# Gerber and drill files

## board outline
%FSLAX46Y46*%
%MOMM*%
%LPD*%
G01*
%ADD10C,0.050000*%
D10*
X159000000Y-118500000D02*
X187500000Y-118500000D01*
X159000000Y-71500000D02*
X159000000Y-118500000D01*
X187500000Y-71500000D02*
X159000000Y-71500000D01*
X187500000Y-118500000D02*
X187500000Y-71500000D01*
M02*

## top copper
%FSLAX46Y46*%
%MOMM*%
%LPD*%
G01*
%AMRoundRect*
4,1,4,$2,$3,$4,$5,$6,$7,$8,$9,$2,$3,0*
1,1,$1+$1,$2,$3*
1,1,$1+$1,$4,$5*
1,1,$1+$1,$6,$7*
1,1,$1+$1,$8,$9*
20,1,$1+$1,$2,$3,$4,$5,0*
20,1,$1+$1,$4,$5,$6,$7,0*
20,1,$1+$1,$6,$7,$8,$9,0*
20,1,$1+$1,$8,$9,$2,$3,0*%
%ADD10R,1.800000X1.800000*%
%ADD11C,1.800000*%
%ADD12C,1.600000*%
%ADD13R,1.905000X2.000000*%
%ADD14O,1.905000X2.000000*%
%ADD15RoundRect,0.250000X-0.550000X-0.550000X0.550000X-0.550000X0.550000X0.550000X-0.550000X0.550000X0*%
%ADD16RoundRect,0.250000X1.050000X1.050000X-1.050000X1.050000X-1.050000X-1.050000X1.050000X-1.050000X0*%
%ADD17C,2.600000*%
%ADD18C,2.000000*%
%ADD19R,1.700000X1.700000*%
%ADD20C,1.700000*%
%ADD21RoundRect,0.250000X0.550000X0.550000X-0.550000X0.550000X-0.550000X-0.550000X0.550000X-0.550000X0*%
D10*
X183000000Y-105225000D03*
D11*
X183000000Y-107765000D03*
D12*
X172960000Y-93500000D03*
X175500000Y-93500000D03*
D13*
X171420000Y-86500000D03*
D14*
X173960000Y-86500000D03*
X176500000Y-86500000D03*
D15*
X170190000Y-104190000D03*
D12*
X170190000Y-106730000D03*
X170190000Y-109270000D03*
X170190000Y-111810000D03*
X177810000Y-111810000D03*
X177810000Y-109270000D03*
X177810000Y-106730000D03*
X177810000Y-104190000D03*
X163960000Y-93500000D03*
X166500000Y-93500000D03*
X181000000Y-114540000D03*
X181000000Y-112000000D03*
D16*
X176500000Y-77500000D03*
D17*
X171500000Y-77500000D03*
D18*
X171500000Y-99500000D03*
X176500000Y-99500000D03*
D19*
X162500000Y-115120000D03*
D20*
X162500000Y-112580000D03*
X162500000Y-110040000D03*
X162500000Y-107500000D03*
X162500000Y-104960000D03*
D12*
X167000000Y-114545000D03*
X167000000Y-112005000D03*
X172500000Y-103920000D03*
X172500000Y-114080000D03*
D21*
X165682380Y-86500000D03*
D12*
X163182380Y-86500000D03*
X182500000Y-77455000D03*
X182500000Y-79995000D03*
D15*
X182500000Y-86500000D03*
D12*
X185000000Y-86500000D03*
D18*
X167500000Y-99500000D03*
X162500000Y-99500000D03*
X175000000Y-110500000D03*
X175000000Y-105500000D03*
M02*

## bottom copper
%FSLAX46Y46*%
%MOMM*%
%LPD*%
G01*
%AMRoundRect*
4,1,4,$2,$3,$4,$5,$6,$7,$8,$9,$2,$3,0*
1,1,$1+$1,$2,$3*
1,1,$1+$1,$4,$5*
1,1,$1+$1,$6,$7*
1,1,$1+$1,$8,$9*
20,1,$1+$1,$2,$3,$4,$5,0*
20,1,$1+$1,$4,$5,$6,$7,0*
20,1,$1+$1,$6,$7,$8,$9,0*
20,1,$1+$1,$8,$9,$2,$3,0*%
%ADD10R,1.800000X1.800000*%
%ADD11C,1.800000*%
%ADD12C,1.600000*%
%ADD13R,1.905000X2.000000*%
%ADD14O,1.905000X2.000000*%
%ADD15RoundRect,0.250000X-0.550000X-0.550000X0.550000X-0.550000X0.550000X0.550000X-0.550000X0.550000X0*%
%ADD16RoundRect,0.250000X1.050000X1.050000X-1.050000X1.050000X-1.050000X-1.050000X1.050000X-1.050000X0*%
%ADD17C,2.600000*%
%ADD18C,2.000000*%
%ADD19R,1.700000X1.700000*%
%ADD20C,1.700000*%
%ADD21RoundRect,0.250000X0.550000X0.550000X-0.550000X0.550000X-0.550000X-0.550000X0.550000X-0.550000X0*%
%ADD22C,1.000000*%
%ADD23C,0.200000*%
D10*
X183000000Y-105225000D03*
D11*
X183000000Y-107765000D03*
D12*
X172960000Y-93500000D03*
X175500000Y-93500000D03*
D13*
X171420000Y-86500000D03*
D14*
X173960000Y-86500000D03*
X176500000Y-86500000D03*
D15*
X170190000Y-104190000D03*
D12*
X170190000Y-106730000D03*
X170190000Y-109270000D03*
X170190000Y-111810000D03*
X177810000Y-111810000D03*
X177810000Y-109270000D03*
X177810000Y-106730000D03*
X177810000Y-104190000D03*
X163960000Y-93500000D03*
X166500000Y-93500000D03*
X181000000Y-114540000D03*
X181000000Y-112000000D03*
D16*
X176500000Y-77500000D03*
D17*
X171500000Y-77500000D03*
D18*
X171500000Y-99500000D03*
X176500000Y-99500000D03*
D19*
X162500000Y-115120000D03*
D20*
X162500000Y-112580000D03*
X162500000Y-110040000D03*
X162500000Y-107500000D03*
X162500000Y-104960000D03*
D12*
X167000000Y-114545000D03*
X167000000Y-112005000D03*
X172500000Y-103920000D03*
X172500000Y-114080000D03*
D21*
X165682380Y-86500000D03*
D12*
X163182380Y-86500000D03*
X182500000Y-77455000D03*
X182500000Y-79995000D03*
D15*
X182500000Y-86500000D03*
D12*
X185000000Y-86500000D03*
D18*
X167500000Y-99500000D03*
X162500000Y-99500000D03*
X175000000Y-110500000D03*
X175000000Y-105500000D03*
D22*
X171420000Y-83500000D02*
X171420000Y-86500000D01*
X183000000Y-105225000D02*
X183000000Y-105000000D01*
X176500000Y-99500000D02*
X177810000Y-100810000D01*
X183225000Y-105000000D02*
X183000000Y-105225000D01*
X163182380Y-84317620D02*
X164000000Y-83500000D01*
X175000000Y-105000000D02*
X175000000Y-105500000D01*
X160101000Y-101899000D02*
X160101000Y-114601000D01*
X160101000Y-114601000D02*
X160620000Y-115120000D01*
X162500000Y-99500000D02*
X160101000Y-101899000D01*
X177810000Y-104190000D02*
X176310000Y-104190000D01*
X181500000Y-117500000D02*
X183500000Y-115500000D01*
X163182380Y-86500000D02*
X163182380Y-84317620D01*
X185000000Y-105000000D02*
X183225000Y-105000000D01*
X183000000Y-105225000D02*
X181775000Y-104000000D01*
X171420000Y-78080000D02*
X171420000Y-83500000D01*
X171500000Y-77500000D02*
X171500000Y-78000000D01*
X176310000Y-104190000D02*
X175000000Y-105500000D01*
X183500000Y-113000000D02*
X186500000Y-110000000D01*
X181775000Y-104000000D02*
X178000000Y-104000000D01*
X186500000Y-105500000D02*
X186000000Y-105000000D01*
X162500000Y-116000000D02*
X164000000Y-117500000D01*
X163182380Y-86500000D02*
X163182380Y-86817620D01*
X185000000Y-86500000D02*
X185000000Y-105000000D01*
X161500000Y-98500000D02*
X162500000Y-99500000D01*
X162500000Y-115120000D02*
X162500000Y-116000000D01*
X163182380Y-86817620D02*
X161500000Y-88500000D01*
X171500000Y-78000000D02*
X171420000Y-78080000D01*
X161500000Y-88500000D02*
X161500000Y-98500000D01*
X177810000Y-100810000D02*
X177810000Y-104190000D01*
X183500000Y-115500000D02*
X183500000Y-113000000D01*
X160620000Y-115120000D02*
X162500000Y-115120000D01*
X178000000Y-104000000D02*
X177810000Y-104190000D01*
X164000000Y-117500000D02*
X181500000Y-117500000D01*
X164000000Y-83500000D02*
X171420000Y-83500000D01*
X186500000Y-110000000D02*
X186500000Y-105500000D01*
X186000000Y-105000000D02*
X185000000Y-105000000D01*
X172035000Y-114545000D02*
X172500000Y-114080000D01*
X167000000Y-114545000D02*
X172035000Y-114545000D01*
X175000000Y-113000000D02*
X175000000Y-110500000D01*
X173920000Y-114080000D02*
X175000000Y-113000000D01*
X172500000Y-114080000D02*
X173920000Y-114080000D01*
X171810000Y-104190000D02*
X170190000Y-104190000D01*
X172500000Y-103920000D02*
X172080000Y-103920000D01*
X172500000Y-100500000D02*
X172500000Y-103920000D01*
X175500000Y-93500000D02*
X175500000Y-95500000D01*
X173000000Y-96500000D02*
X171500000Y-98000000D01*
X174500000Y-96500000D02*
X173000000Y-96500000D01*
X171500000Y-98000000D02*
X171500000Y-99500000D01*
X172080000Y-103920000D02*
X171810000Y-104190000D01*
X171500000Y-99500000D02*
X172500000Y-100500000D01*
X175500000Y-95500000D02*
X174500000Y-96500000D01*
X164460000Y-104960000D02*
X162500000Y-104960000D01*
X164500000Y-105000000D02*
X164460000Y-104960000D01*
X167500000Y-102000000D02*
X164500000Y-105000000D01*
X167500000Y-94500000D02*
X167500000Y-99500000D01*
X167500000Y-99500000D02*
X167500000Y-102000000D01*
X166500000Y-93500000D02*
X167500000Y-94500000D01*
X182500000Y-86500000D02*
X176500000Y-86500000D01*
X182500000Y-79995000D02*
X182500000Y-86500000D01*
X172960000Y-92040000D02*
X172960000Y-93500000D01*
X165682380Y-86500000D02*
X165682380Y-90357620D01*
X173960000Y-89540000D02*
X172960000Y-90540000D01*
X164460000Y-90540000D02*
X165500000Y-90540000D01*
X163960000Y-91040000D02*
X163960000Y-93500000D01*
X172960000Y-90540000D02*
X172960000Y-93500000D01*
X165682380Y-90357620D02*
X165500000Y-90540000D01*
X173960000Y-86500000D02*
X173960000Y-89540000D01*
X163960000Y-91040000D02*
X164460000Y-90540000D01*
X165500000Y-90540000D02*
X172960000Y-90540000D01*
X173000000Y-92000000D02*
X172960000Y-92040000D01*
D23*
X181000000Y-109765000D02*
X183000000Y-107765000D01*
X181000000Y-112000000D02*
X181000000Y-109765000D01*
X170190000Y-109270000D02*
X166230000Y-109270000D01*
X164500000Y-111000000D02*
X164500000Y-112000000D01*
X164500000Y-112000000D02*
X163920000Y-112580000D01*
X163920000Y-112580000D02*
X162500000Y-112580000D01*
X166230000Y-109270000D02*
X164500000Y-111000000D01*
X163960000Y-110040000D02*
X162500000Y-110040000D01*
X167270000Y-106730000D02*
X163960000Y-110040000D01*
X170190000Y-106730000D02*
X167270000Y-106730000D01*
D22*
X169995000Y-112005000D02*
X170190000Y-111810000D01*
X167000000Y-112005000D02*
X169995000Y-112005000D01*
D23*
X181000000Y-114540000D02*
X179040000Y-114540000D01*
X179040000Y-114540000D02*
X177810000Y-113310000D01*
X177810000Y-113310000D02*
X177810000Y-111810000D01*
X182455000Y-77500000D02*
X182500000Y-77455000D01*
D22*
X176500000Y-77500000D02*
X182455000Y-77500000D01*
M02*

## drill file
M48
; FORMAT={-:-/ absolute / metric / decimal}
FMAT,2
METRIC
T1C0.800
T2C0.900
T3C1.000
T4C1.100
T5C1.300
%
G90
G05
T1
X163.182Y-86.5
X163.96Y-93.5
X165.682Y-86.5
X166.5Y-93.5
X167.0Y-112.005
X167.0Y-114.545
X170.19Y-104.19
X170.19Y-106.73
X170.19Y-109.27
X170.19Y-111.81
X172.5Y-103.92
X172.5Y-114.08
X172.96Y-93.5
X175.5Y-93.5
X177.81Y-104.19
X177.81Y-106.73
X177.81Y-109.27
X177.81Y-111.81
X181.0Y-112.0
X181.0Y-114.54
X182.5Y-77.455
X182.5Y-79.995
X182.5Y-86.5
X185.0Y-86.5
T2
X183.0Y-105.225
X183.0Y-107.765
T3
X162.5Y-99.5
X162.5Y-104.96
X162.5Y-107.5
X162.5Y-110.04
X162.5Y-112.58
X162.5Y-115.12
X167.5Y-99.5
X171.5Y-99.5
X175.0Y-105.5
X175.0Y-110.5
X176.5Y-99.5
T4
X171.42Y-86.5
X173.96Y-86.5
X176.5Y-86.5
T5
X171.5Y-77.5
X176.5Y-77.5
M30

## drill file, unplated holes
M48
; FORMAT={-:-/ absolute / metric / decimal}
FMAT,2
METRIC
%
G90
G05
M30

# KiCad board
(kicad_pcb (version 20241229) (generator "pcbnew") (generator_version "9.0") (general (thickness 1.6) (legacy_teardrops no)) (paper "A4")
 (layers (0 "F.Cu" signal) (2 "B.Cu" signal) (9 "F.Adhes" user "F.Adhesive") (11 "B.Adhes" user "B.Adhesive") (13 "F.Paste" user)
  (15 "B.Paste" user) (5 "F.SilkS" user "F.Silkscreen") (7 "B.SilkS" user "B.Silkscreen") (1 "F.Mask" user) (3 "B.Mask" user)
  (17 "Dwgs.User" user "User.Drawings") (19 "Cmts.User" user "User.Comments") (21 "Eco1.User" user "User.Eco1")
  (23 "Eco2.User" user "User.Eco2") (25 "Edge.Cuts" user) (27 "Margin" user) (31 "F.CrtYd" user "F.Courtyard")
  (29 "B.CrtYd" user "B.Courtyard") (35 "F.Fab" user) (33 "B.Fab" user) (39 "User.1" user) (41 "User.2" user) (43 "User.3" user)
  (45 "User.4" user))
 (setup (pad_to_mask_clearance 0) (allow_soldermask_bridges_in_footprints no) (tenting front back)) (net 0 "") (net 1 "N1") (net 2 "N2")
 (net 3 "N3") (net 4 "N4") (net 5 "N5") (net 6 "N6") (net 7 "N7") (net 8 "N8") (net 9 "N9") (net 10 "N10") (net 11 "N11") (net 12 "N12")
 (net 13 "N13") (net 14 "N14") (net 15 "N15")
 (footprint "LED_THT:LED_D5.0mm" (layer "F.Cu") (at 183 105.225 -90)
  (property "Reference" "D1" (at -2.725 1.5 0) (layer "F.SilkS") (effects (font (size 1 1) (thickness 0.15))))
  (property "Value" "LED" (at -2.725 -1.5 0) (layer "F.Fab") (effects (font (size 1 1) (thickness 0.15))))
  (pad "1" thru_hole rect (at 0 0 270) (size 1.8 1.8) (drill 0.9) (layers "*.Cu" "*.Mask") (remove_unused_layers no) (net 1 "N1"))
  (pad "2" thru_hole circle (at 2.54 0 270) (size 1.8 1.8) (drill 0.9) (layers "*.Cu" "*.Mask") (remove_unused_layers no) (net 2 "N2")))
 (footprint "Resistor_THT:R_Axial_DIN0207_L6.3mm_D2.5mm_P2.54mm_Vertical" (layer "F.Cu") (at 172.96 93.5)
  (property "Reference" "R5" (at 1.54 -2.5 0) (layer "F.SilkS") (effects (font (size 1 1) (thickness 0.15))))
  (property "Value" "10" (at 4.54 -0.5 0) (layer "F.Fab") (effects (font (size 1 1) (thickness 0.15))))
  (pad "1" thru_hole circle (at 0 0) (size 1.6 1.6) (drill 0.8) (layers "*.Cu" "*.Mask") (remove_unused_layers no) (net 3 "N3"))
  (pad "2" thru_hole circle (at 2.54 0) (size 1.6 1.6) (drill 0.8) (layers "*.Cu" "*.Mask") (remove_unused_layers no) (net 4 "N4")))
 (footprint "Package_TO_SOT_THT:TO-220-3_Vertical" (layer "F.Cu") (at 171.42 86.5)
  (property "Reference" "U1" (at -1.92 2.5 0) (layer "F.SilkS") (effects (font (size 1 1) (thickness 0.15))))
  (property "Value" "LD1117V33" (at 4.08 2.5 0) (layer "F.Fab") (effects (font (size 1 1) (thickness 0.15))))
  (pad "1" thru_hole rect (at 0 0) (size 1.905 2) (drill 1.1) (layers "*.Cu" "*.Mask") (remove_unused_layers no) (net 1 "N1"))
  (pad "2" thru_hole oval (at 2.54 0) (size 1.905 2) (drill 1.1) (layers "*.Cu" "*.Mask") (remove_unused_layers no) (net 3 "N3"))
  (pad "3" thru_hole oval (at 5.08 0) (size 1.905 2) (drill 1.1) (layers "*.Cu" "*.Mask") (remove_unused_layers no) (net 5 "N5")))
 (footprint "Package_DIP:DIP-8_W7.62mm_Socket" (layer "F.Cu") (at 170.19 104.19)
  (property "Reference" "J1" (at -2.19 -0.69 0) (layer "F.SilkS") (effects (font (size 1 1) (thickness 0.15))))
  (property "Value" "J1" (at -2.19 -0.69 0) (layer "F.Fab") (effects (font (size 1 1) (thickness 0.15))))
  (pad "1" thru_hole roundrect (at 0 0) (size 1.6 1.6) (drill 0.8) (layers "*.Cu" "*.Mask") (remove_unused_layers no)
   (roundrect_rratio 0.15625) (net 4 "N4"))
  (pad "2" thru_hole circle (at 0 2.54) (size 1.6 1.6) (drill 0.8) (layers "*.Cu" "*.Mask") (remove_unused_layers no) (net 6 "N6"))
  (pad "3" thru_hole circle (at 0 5.08) (size 1.6 1.6) (drill 0.8) (layers "*.Cu" "*.Mask") (remove_unused_layers no) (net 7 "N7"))
  (pad "4" thru_hole circle (at 0 7.62) (size 1.6 1.6) (drill 0.8) (layers "*.Cu" "*.Mask") (remove_unused_layers no) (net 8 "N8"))
  (pad "5" thru_hole circle (at 7.62 7.62) (size 1.6 1.6) (drill 0.8) (layers "*.Cu" "*.Mask") (remove_unused_layers no) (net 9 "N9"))
  (pad "6" thru_hole circle (at 7.62 5.08) (size 1.6 1.6) (drill 0.8) (layers "*.Cu" "*.Mask") (remove_unused_layers no) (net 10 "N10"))
  (pad "7" thru_hole circle (at 7.62 2.54) (size 1.6 1.6) (drill 0.8) (layers "*.Cu" "*.Mask") (remove_unused_layers no) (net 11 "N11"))
  (pad "8" thru_hole circle (at 7.62 0) (size 1.6 1.6) (drill 0.8) (layers "*.Cu" "*.Mask") (remove_unused_layers no) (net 1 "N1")))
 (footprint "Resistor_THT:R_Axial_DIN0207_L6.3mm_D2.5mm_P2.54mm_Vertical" (layer "F.Cu") (at 163.96 93.5)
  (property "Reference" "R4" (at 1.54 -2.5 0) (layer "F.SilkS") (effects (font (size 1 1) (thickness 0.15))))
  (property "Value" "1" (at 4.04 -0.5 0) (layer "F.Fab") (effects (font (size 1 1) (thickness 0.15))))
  (pad "1" thru_hole circle (at 0 0) (size 1.6 1.6) (drill 0.8) (layers "*.Cu" "*.Mask") (remove_unused_layers no) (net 3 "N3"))
  (pad "2" thru_hole circle (at 2.54 0) (size 1.6 1.6) (drill 0.8) (layers "*.Cu" "*.Mask") (remove_unused_layers no) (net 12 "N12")))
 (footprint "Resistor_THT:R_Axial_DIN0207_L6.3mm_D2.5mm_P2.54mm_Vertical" (layer "F.Cu") (at 181 114.54 90)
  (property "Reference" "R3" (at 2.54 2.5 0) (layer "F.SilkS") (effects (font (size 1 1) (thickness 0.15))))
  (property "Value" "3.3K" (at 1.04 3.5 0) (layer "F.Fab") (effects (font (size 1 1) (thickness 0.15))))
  (pad "1" thru_hole circle (at 0 0 90) (size 1.6 1.6) (drill 0.8) (layers "*.Cu" "*.Mask") (remove_unused_layers no) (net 9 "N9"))
  (pad "2" thru_hole circle (at 2.54 0 90) (size 1.6 1.6) (drill 0.8) (layers "*.Cu" "*.Mask") (remove_unused_layers no) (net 2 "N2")))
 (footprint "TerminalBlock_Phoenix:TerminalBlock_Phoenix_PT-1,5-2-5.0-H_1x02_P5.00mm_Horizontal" (layer "F.Cu") (at 176.5 77.5 180)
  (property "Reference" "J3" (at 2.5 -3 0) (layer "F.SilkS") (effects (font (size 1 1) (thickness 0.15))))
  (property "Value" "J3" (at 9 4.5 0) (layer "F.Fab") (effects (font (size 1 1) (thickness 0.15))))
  (pad "1" thru_hole roundrect (at 0 0 180) (size 2.6 2.6) (drill 1.3) (layers "*.Cu" "*.Mask") (remove_unused_layers no)
   (roundrect_rratio 0.096154) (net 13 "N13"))
  (pad "2" thru_hole circle (at 5 0 180) (size 2.6 2.6) (drill 1.3) (layers "*.Cu" "*.Mask") (remove_unused_layers no) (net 1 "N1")))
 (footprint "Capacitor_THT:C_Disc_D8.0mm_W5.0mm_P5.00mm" (layer "F.Cu") (at 171.5 99.5)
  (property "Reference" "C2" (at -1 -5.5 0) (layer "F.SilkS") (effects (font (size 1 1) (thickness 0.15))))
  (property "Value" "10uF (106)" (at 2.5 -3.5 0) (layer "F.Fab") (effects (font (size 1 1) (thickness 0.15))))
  (pad "1" thru_hole circle (at 0 0) (size 2 2) (drill 1) (layers "*.Cu" "*.Mask") (remove_unused_layers no) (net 4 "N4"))
  (pad "2" thru_hole circle (at 5 0) (size 2 2) (drill 1) (layers "*.Cu" "*.Mask") (remove_unused_layers no) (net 1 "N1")))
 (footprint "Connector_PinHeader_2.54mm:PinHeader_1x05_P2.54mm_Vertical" (layer "F.Cu") (at 162.5 115.12 180)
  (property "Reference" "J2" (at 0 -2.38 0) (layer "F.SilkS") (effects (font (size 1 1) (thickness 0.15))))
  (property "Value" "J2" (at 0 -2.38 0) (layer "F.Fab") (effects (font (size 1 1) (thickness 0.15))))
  (pad "1" thru_hole rect (at 0 0 180) (size 1.7 1.7) (drill 1) (layers "*.Cu" "*.Mask") (remove_unused_layers no) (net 1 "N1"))
  (pad "2" thru_hole circle (at 0 2.54 180) (size 1.7 1.7) (drill 1) (layers "*.Cu" "*.Mask") (remove_unused_layers no) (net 7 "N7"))
  (pad "3" thru_hole circle (at 0 5.08 180) (size 1.7 1.7) (drill 1) (layers "*.Cu" "*.Mask") (remove_unused_layers no) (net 6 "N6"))
  (pad "4" thru_hole circle (at 0 7.62 180) (size 1.7 1.7) (drill 1) (layers "*.Cu" "*.Mask") (remove_unused_layers no) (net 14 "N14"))
  (pad "5" thru_hole circle (at 0 10.16 180) (size 1.7 1.7) (drill 1) (layers "*.Cu" "*.Mask") (remove_unused_layers no) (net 12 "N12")))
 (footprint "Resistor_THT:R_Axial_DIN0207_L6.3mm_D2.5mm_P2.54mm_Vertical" (layer "F.Cu") (at 167 114.545 90)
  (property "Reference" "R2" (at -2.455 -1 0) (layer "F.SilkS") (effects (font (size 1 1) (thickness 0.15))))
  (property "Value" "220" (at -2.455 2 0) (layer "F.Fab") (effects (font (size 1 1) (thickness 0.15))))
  (pad "1" thru_hole circle (at 0 0 90) (size 1.6 1.6) (drill 0.8) (layers "*.Cu" "*.Mask") (remove_unused_layers no) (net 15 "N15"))
  (pad "2" thru_hole circle (at 2.54 0 90) (size 1.6 1.6) (drill 0.8) (layers "*.Cu" "*.Mask") (remove_unused_layers no) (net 8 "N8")))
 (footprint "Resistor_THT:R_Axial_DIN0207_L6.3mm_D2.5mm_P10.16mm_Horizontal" (layer "F.Cu") (at 172.5 103.92 -90)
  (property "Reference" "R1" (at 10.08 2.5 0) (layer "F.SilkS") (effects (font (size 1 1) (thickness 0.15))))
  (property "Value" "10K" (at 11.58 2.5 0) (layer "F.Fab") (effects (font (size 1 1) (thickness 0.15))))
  (pad "1" thru_hole circle (at 0 0 270) (size 1.6 1.6) (drill 0.8) (layers "*.Cu" "*.Mask") (remove_unused_layers no) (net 4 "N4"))
  (pad "2" thru_hole circle (at 10.16 0 270) (size 1.6 1.6) (drill 0.8) (layers "*.Cu" "*.Mask") (remove_unused_layers no) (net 15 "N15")))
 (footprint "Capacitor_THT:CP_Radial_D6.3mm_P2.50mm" (layer "F.Cu") (at 165.68238 86.5 180)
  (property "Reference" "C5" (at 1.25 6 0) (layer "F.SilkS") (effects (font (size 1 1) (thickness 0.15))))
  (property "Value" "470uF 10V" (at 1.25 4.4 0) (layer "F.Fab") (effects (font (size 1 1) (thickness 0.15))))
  (pad "1" thru_hole roundrect (at 0 0 180) (size 1.6 1.6) (drill 0.8) (layers "*.Cu" "*.Mask") (remove_unused_layers no)
   (roundrect_rratio 0.15625) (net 3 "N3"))
  (pad "2" thru_hole circle (at 2.5 0 180) (size 1.6 1.6) (drill 0.8) (layers "*.Cu" "*.Mask") (remove_unused_layers no) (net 1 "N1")))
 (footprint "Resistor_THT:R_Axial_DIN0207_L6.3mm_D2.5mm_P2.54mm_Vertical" (layer "F.Cu") (at 182.5 77.455 -90)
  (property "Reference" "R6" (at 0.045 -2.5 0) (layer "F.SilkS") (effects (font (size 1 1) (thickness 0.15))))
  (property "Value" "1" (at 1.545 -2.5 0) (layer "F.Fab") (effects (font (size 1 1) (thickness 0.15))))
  (pad "1" thru_hole circle (at 0 0 270) (size 1.6 1.6) (drill 0.8) (layers "*.Cu" "*.Mask") (remove_unused_layers no) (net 13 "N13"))
  (pad "2" thru_hole circle (at 2.54 0 270) (size 1.6 1.6) (drill 0.8) (layers "*.Cu" "*.Mask") (remove_unused_layers no) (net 5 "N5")))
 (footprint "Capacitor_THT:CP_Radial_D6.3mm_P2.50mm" (layer "F.Cu") (at 182.5 86.5)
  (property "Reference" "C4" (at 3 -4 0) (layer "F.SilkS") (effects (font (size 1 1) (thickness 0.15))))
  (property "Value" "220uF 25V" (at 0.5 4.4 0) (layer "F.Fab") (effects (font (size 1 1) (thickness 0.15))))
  (pad "1" thru_hole roundrect (at 0 0) (size 1.6 1.6) (drill 0.8) (layers "*.Cu" "*.Mask") (remove_unused_layers no)
   (roundrect_rratio 0.15625) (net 5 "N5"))
  (pad "2" thru_hole circle (at 2.5 0) (size 1.6 1.6) (drill 0.8) (layers "*.Cu" "*.Mask") (remove_unused_layers no) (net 1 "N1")))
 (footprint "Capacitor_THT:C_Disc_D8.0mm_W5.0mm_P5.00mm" (layer "F.Cu") (at 167.5 99.5 180)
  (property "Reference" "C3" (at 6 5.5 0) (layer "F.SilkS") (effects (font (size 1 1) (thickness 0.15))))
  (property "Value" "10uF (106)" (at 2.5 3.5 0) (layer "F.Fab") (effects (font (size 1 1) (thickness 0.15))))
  (pad "1" thru_hole circle (at 0 0 180) (size 2 2) (drill 1) (layers "*.Cu" "*.Mask") (remove_unused_layers no) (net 12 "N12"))
  (pad "2" thru_hole circle (at 5 0 180) (size 2 2) (drill 1) (layers "*.Cu" "*.Mask") (remove_unused_layers no) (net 1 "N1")))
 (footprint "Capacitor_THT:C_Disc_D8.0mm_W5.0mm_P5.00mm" (layer "F.Cu") (at 175 110.5 90)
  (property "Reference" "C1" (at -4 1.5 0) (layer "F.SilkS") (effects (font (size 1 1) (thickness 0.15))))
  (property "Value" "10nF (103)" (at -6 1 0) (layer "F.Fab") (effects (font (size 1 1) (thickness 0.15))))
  (pad "1" thru_hole circle (at 0 0 90) (size 2 2) (drill 1) (layers "*.Cu" "*.Mask") (remove_unused_layers no) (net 15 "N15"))
  (pad "2" thru_hole circle (at 5 0 90) (size 2 2) (drill 1) (layers "*.Cu" "*.Mask") (remove_unused_layers no) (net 1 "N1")))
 (gr_line (start 159 118.5) (end 187.5 118.5) (stroke (width 0.05) (type default)) (layer "Edge.Cuts"))
 (gr_line (start 159 71.5) (end 159 118.5) (stroke (width 0.05) (type default)) (layer "Edge.Cuts"))
 (gr_line (start 187.5 71.5) (end 159 71.5) (stroke (width 0.05) (type default)) (layer "Edge.Cuts"))
 (gr_line (start 187.5 118.5) (end 187.5 71.5) (stroke (width 0.05) (type default)) (layer "Edge.Cuts"))
 (segment (start 171.42 83.5) (end 171.42 86.5) (width 1) (layer "B.Cu") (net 1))
 (segment (start 183 105.225) (end 183 105) (width 1) (layer "B.Cu") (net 1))
 (segment (start 176.5 99.5) (end 177.81 100.81) (width 1) (layer "B.Cu") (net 1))
 (segment (start 183.225 105) (end 183 105.225) (width 1) (layer "B.Cu") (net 1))
 (segment (start 163.18238 84.31762) (end 164 83.5) (width 1) (layer "B.Cu") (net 1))
 (segment (start 175 105) (end 175 105.5) (width 1) (layer "B.Cu") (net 1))
 (segment (start 160.101 101.899) (end 160.101 114.601) (width 1) (layer "B.Cu") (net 1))
 (segment (start 160.101 114.601) (end 160.62 115.12) (width 1) (layer "B.Cu") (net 1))
 (segment (start 162.5 99.5) (end 160.101 101.899) (width 1) (layer "B.Cu") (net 1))
 (segment (start 177.81 104.19) (end 176.31 104.19) (width 1) (layer "B.Cu") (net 1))
 (segment (start 181.5 117.5) (end 183.5 115.5) (width 1) (layer "B.Cu") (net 1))
 (segment (start 163.18238 86.5) (end 163.18238 84.31762) (width 1) (layer "B.Cu") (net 1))
 (segment (start 185 105) (end 183.225 105) (width 1) (layer "B.Cu") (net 1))
 (segment (start 183 105.225) (end 181.775 104) (width 1) (layer "B.Cu") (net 1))
 (segment (start 171.42 78.08) (end 171.42 83.5) (width 1) (layer "B.Cu") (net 1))
 (segment (start 171.5 77.5) (end 171.5 78) (width 1) (layer "B.Cu") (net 1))
 (segment (start 176.31 104.19) (end 175 105.5) (width 1) (layer "B.Cu") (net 1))
 (segment (start 183.5 113) (end 186.5 110) (width 1) (layer "B.Cu") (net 1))
 (segment (start 181.775 104) (end 178 104) (width 1) (layer "B.Cu") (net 1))
 (segment (start 186.5 105.5) (end 186 105) (width 1) (layer "B.Cu") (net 1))
 (segment (start 162.5 116) (end 164 117.5) (width 1) (layer "B.Cu") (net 1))
 (segment (start 163.18238 86.5) (end 163.18238 86.81762) (width 1) (layer "B.Cu") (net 1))
 (segment (start 185 86.5) (end 185 105) (width 1) (layer "B.Cu") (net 1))
 (segment (start 161.5 98.5) (end 162.5 99.5) (width 1) (layer "B.Cu") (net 1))
 (segment (start 162.5 115.12) (end 162.5 116) (width 1) (layer "B.Cu") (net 1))
 (segment (start 163.18238 86.81762) (end 161.5 88.5) (width 1) (layer "B.Cu") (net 1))
 (segment (start 171.5 78) (end 171.42 78.08) (width 1) (layer "B.Cu") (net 1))
 (segment (start 161.5 88.5) (end 161.5 98.5) (width 1) (layer "B.Cu") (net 1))
 (segment (start 177.81 100.81) (end 177.81 104.19) (width 1) (layer "B.Cu") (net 1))
 (segment (start 183.5 115.5) (end 183.5 113) (width 1) (layer "B.Cu") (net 1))
 (segment (start 160.62 115.12) (end 162.5 115.12) (width 1) (layer "B.Cu") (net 1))
 (segment (start 178 104) (end 177.81 104.19) (width 1) (layer "B.Cu") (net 1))
 (segment (start 164 117.5) (end 181.5 117.5) (width 1) (layer "B.Cu") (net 1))
 (segment (start 164 83.5) (end 171.42 83.5) (width 1) (layer "B.Cu") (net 1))
 (segment (start 186.5 110) (end 186.5 105.5) (width 1) (layer "B.Cu") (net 1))
 (segment (start 186 105) (end 185 105) (width 1) (layer "B.Cu") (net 1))
 (segment (start 172.035 114.545) (end 172.5 114.08) (width 1) (layer "B.Cu") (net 15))
 (segment (start 167 114.545) (end 172.035 114.545) (width 1) (layer "B.Cu") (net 15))
 (segment (start 175 113) (end 175 110.5) (width 1) (layer "B.Cu") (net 15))
 (segment (start 173.92 114.08) (end 175 113) (width 1) (layer "B.Cu") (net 15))
 (segment (start 172.5 114.08) (end 173.92 114.08) (width 1) (layer "B.Cu") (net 15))
 (segment (start 171.81 104.19) (end 170.19 104.19) (width 1) (layer "B.Cu") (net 4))
 (segment (start 172.5 103.92) (end 172.08 103.92) (width 1) (layer "B.Cu") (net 4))
 (segment (start 172.5 100.5) (end 172.5 103.92) (width 1) (layer "B.Cu") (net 4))
 (segment (start 175.5 93.5) (end 175.5 95.5) (width 1) (layer "B.Cu") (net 4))
 (segment (start 173 96.5) (end 171.5 98) (width 1) (layer "B.Cu") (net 4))
 (segment (start 174.5 96.5) (end 173 96.5) (width 1) (layer "B.Cu") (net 4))
 (segment (start 171.5 98) (end 171.5 99.5) (width 1) (layer "B.Cu") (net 4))
 (segment (start 172.08 103.92) (end 171.81 104.19) (width 1) (layer "B.Cu") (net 4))
 (segment (start 171.5 99.5) (end 172.5 100.5) (width 1) (layer "B.Cu") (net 4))
 (segment (start 175.5 95.5) (end 174.5 96.5) (width 1) (layer "B.Cu") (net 4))
 (segment (start 164.46 104.96) (end 162.5 104.96) (width 1) (layer "B.Cu") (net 12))
 (segment (start 164.5 105) (end 164.46 104.96) (width 1) (layer "B.Cu") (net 12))
 (segment (start 167.5 102) (end 164.5 105) (width 1) (layer "B.Cu") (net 12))
 (segment (start 167.5 94.5) (end 167.5 99.5) (width 1) (layer "B.Cu") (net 12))
 (segment (start 167.5 99.5) (end 167.5 102) (width 1) (layer "B.Cu") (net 12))
 (segment (start 166.5 93.5) (end 167.5 94.5) (width 1) (layer "B.Cu") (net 12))
 (segment (start 182.5 86.5) (end 176.5 86.5) (width 1) (layer "B.Cu") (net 5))
 (segment (start 182.5 79.995) (end 182.5 86.5) (width 1) (layer "B.Cu") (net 5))
 (segment (start 172.96 92.04) (end 172.96 93.5) (width 1) (layer "B.Cu") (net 3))
 (segment (start 165.68238 86.5) (end 165.68238 90.35762) (width 1) (layer "B.Cu") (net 3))
 (segment (start 173.96 89.54) (end 172.96 90.54) (width 1) (layer "B.Cu") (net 3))
 (segment (start 164.46 90.54) (end 165.5 90.54) (width 1) (layer "B.Cu") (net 3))
 (segment (start 163.96 91.04) (end 163.96 93.5) (width 1) (layer "B.Cu") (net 3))
 (segment (start 172.96 90.54) (end 172.96 93.5) (width 1) (layer "B.Cu") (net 3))
 (segment (start 165.68238 90.35762) (end 165.5 90.54) (width 1) (layer "B.Cu") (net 3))
 (segment (start 173.96 86.5) (end 173.96 89.54) (width 1) (layer "B.Cu") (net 3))
 (segment (start 163.96 91.04) (end 164.46 90.54) (width 1) (layer "B.Cu") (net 3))
 (segment (start 165.5 90.54) (end 172.96 90.54) (width 1) (layer "B.Cu") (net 3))
 (segment (start 173 92) (end 172.96 92.04) (width 1) (layer "B.Cu") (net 3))
 (segment (start 181 109.765) (end 183 107.765) (width 0.2) (layer "B.Cu") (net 2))
 (segment (start 181 112) (end 181 109.765) (width 0.2) (layer "B.Cu") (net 2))
 (segment (start 170.19 109.27) (end 166.23 109.27) (width 0.2) (layer "B.Cu") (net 7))
 (segment (start 164.5 111) (end 164.5 112) (width 0.2) (layer "B.Cu") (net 7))
 (segment (start 164.5 112) (end 163.92 112.58) (width 0.2) (layer "B.Cu") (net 7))
 (segment (start 163.92 112.58) (end 162.5 112.58) (width 0.2) (layer "B.Cu") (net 7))
 (segment (start 166.23 109.27) (end 164.5 111) (width 0.2) (layer "B.Cu") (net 7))
 (segment (start 163.96 110.04) (end 162.5 110.04) (width 0.2) (layer "B.Cu") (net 6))
 (segment (start 167.27 106.73) (end 163.96 110.04) (width 0.2) (layer "B.Cu") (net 6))
 (segment (start 170.19 106.73) (end 167.27 106.73) (width 0.2) (layer "B.Cu") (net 6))
 (segment (start 169.995 112.005) (end 170.19 111.81) (width 1) (layer "B.Cu") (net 8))
 (segment (start 167 112.005) (end 169.995 112.005) (width 1) (layer "B.Cu") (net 8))
 (segment (start 181 114.54) (end 179.04 114.54) (width 0.2) (layer "B.Cu") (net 9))
 (segment (start 179.04 114.54) (end 177.81 113.31) (width 0.2) (layer "B.Cu") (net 9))
 (segment (start 177.81 113.31) (end 177.81 111.81) (width 0.2) (layer "B.Cu") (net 9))
 (segment (start 182.455 77.5) (end 182.5 77.455) (width 0.2) (layer "B.Cu") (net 13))
 (segment (start 176.5 77.5) (end 182.455 77.5) (width 1) (layer "B.Cu") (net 13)))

